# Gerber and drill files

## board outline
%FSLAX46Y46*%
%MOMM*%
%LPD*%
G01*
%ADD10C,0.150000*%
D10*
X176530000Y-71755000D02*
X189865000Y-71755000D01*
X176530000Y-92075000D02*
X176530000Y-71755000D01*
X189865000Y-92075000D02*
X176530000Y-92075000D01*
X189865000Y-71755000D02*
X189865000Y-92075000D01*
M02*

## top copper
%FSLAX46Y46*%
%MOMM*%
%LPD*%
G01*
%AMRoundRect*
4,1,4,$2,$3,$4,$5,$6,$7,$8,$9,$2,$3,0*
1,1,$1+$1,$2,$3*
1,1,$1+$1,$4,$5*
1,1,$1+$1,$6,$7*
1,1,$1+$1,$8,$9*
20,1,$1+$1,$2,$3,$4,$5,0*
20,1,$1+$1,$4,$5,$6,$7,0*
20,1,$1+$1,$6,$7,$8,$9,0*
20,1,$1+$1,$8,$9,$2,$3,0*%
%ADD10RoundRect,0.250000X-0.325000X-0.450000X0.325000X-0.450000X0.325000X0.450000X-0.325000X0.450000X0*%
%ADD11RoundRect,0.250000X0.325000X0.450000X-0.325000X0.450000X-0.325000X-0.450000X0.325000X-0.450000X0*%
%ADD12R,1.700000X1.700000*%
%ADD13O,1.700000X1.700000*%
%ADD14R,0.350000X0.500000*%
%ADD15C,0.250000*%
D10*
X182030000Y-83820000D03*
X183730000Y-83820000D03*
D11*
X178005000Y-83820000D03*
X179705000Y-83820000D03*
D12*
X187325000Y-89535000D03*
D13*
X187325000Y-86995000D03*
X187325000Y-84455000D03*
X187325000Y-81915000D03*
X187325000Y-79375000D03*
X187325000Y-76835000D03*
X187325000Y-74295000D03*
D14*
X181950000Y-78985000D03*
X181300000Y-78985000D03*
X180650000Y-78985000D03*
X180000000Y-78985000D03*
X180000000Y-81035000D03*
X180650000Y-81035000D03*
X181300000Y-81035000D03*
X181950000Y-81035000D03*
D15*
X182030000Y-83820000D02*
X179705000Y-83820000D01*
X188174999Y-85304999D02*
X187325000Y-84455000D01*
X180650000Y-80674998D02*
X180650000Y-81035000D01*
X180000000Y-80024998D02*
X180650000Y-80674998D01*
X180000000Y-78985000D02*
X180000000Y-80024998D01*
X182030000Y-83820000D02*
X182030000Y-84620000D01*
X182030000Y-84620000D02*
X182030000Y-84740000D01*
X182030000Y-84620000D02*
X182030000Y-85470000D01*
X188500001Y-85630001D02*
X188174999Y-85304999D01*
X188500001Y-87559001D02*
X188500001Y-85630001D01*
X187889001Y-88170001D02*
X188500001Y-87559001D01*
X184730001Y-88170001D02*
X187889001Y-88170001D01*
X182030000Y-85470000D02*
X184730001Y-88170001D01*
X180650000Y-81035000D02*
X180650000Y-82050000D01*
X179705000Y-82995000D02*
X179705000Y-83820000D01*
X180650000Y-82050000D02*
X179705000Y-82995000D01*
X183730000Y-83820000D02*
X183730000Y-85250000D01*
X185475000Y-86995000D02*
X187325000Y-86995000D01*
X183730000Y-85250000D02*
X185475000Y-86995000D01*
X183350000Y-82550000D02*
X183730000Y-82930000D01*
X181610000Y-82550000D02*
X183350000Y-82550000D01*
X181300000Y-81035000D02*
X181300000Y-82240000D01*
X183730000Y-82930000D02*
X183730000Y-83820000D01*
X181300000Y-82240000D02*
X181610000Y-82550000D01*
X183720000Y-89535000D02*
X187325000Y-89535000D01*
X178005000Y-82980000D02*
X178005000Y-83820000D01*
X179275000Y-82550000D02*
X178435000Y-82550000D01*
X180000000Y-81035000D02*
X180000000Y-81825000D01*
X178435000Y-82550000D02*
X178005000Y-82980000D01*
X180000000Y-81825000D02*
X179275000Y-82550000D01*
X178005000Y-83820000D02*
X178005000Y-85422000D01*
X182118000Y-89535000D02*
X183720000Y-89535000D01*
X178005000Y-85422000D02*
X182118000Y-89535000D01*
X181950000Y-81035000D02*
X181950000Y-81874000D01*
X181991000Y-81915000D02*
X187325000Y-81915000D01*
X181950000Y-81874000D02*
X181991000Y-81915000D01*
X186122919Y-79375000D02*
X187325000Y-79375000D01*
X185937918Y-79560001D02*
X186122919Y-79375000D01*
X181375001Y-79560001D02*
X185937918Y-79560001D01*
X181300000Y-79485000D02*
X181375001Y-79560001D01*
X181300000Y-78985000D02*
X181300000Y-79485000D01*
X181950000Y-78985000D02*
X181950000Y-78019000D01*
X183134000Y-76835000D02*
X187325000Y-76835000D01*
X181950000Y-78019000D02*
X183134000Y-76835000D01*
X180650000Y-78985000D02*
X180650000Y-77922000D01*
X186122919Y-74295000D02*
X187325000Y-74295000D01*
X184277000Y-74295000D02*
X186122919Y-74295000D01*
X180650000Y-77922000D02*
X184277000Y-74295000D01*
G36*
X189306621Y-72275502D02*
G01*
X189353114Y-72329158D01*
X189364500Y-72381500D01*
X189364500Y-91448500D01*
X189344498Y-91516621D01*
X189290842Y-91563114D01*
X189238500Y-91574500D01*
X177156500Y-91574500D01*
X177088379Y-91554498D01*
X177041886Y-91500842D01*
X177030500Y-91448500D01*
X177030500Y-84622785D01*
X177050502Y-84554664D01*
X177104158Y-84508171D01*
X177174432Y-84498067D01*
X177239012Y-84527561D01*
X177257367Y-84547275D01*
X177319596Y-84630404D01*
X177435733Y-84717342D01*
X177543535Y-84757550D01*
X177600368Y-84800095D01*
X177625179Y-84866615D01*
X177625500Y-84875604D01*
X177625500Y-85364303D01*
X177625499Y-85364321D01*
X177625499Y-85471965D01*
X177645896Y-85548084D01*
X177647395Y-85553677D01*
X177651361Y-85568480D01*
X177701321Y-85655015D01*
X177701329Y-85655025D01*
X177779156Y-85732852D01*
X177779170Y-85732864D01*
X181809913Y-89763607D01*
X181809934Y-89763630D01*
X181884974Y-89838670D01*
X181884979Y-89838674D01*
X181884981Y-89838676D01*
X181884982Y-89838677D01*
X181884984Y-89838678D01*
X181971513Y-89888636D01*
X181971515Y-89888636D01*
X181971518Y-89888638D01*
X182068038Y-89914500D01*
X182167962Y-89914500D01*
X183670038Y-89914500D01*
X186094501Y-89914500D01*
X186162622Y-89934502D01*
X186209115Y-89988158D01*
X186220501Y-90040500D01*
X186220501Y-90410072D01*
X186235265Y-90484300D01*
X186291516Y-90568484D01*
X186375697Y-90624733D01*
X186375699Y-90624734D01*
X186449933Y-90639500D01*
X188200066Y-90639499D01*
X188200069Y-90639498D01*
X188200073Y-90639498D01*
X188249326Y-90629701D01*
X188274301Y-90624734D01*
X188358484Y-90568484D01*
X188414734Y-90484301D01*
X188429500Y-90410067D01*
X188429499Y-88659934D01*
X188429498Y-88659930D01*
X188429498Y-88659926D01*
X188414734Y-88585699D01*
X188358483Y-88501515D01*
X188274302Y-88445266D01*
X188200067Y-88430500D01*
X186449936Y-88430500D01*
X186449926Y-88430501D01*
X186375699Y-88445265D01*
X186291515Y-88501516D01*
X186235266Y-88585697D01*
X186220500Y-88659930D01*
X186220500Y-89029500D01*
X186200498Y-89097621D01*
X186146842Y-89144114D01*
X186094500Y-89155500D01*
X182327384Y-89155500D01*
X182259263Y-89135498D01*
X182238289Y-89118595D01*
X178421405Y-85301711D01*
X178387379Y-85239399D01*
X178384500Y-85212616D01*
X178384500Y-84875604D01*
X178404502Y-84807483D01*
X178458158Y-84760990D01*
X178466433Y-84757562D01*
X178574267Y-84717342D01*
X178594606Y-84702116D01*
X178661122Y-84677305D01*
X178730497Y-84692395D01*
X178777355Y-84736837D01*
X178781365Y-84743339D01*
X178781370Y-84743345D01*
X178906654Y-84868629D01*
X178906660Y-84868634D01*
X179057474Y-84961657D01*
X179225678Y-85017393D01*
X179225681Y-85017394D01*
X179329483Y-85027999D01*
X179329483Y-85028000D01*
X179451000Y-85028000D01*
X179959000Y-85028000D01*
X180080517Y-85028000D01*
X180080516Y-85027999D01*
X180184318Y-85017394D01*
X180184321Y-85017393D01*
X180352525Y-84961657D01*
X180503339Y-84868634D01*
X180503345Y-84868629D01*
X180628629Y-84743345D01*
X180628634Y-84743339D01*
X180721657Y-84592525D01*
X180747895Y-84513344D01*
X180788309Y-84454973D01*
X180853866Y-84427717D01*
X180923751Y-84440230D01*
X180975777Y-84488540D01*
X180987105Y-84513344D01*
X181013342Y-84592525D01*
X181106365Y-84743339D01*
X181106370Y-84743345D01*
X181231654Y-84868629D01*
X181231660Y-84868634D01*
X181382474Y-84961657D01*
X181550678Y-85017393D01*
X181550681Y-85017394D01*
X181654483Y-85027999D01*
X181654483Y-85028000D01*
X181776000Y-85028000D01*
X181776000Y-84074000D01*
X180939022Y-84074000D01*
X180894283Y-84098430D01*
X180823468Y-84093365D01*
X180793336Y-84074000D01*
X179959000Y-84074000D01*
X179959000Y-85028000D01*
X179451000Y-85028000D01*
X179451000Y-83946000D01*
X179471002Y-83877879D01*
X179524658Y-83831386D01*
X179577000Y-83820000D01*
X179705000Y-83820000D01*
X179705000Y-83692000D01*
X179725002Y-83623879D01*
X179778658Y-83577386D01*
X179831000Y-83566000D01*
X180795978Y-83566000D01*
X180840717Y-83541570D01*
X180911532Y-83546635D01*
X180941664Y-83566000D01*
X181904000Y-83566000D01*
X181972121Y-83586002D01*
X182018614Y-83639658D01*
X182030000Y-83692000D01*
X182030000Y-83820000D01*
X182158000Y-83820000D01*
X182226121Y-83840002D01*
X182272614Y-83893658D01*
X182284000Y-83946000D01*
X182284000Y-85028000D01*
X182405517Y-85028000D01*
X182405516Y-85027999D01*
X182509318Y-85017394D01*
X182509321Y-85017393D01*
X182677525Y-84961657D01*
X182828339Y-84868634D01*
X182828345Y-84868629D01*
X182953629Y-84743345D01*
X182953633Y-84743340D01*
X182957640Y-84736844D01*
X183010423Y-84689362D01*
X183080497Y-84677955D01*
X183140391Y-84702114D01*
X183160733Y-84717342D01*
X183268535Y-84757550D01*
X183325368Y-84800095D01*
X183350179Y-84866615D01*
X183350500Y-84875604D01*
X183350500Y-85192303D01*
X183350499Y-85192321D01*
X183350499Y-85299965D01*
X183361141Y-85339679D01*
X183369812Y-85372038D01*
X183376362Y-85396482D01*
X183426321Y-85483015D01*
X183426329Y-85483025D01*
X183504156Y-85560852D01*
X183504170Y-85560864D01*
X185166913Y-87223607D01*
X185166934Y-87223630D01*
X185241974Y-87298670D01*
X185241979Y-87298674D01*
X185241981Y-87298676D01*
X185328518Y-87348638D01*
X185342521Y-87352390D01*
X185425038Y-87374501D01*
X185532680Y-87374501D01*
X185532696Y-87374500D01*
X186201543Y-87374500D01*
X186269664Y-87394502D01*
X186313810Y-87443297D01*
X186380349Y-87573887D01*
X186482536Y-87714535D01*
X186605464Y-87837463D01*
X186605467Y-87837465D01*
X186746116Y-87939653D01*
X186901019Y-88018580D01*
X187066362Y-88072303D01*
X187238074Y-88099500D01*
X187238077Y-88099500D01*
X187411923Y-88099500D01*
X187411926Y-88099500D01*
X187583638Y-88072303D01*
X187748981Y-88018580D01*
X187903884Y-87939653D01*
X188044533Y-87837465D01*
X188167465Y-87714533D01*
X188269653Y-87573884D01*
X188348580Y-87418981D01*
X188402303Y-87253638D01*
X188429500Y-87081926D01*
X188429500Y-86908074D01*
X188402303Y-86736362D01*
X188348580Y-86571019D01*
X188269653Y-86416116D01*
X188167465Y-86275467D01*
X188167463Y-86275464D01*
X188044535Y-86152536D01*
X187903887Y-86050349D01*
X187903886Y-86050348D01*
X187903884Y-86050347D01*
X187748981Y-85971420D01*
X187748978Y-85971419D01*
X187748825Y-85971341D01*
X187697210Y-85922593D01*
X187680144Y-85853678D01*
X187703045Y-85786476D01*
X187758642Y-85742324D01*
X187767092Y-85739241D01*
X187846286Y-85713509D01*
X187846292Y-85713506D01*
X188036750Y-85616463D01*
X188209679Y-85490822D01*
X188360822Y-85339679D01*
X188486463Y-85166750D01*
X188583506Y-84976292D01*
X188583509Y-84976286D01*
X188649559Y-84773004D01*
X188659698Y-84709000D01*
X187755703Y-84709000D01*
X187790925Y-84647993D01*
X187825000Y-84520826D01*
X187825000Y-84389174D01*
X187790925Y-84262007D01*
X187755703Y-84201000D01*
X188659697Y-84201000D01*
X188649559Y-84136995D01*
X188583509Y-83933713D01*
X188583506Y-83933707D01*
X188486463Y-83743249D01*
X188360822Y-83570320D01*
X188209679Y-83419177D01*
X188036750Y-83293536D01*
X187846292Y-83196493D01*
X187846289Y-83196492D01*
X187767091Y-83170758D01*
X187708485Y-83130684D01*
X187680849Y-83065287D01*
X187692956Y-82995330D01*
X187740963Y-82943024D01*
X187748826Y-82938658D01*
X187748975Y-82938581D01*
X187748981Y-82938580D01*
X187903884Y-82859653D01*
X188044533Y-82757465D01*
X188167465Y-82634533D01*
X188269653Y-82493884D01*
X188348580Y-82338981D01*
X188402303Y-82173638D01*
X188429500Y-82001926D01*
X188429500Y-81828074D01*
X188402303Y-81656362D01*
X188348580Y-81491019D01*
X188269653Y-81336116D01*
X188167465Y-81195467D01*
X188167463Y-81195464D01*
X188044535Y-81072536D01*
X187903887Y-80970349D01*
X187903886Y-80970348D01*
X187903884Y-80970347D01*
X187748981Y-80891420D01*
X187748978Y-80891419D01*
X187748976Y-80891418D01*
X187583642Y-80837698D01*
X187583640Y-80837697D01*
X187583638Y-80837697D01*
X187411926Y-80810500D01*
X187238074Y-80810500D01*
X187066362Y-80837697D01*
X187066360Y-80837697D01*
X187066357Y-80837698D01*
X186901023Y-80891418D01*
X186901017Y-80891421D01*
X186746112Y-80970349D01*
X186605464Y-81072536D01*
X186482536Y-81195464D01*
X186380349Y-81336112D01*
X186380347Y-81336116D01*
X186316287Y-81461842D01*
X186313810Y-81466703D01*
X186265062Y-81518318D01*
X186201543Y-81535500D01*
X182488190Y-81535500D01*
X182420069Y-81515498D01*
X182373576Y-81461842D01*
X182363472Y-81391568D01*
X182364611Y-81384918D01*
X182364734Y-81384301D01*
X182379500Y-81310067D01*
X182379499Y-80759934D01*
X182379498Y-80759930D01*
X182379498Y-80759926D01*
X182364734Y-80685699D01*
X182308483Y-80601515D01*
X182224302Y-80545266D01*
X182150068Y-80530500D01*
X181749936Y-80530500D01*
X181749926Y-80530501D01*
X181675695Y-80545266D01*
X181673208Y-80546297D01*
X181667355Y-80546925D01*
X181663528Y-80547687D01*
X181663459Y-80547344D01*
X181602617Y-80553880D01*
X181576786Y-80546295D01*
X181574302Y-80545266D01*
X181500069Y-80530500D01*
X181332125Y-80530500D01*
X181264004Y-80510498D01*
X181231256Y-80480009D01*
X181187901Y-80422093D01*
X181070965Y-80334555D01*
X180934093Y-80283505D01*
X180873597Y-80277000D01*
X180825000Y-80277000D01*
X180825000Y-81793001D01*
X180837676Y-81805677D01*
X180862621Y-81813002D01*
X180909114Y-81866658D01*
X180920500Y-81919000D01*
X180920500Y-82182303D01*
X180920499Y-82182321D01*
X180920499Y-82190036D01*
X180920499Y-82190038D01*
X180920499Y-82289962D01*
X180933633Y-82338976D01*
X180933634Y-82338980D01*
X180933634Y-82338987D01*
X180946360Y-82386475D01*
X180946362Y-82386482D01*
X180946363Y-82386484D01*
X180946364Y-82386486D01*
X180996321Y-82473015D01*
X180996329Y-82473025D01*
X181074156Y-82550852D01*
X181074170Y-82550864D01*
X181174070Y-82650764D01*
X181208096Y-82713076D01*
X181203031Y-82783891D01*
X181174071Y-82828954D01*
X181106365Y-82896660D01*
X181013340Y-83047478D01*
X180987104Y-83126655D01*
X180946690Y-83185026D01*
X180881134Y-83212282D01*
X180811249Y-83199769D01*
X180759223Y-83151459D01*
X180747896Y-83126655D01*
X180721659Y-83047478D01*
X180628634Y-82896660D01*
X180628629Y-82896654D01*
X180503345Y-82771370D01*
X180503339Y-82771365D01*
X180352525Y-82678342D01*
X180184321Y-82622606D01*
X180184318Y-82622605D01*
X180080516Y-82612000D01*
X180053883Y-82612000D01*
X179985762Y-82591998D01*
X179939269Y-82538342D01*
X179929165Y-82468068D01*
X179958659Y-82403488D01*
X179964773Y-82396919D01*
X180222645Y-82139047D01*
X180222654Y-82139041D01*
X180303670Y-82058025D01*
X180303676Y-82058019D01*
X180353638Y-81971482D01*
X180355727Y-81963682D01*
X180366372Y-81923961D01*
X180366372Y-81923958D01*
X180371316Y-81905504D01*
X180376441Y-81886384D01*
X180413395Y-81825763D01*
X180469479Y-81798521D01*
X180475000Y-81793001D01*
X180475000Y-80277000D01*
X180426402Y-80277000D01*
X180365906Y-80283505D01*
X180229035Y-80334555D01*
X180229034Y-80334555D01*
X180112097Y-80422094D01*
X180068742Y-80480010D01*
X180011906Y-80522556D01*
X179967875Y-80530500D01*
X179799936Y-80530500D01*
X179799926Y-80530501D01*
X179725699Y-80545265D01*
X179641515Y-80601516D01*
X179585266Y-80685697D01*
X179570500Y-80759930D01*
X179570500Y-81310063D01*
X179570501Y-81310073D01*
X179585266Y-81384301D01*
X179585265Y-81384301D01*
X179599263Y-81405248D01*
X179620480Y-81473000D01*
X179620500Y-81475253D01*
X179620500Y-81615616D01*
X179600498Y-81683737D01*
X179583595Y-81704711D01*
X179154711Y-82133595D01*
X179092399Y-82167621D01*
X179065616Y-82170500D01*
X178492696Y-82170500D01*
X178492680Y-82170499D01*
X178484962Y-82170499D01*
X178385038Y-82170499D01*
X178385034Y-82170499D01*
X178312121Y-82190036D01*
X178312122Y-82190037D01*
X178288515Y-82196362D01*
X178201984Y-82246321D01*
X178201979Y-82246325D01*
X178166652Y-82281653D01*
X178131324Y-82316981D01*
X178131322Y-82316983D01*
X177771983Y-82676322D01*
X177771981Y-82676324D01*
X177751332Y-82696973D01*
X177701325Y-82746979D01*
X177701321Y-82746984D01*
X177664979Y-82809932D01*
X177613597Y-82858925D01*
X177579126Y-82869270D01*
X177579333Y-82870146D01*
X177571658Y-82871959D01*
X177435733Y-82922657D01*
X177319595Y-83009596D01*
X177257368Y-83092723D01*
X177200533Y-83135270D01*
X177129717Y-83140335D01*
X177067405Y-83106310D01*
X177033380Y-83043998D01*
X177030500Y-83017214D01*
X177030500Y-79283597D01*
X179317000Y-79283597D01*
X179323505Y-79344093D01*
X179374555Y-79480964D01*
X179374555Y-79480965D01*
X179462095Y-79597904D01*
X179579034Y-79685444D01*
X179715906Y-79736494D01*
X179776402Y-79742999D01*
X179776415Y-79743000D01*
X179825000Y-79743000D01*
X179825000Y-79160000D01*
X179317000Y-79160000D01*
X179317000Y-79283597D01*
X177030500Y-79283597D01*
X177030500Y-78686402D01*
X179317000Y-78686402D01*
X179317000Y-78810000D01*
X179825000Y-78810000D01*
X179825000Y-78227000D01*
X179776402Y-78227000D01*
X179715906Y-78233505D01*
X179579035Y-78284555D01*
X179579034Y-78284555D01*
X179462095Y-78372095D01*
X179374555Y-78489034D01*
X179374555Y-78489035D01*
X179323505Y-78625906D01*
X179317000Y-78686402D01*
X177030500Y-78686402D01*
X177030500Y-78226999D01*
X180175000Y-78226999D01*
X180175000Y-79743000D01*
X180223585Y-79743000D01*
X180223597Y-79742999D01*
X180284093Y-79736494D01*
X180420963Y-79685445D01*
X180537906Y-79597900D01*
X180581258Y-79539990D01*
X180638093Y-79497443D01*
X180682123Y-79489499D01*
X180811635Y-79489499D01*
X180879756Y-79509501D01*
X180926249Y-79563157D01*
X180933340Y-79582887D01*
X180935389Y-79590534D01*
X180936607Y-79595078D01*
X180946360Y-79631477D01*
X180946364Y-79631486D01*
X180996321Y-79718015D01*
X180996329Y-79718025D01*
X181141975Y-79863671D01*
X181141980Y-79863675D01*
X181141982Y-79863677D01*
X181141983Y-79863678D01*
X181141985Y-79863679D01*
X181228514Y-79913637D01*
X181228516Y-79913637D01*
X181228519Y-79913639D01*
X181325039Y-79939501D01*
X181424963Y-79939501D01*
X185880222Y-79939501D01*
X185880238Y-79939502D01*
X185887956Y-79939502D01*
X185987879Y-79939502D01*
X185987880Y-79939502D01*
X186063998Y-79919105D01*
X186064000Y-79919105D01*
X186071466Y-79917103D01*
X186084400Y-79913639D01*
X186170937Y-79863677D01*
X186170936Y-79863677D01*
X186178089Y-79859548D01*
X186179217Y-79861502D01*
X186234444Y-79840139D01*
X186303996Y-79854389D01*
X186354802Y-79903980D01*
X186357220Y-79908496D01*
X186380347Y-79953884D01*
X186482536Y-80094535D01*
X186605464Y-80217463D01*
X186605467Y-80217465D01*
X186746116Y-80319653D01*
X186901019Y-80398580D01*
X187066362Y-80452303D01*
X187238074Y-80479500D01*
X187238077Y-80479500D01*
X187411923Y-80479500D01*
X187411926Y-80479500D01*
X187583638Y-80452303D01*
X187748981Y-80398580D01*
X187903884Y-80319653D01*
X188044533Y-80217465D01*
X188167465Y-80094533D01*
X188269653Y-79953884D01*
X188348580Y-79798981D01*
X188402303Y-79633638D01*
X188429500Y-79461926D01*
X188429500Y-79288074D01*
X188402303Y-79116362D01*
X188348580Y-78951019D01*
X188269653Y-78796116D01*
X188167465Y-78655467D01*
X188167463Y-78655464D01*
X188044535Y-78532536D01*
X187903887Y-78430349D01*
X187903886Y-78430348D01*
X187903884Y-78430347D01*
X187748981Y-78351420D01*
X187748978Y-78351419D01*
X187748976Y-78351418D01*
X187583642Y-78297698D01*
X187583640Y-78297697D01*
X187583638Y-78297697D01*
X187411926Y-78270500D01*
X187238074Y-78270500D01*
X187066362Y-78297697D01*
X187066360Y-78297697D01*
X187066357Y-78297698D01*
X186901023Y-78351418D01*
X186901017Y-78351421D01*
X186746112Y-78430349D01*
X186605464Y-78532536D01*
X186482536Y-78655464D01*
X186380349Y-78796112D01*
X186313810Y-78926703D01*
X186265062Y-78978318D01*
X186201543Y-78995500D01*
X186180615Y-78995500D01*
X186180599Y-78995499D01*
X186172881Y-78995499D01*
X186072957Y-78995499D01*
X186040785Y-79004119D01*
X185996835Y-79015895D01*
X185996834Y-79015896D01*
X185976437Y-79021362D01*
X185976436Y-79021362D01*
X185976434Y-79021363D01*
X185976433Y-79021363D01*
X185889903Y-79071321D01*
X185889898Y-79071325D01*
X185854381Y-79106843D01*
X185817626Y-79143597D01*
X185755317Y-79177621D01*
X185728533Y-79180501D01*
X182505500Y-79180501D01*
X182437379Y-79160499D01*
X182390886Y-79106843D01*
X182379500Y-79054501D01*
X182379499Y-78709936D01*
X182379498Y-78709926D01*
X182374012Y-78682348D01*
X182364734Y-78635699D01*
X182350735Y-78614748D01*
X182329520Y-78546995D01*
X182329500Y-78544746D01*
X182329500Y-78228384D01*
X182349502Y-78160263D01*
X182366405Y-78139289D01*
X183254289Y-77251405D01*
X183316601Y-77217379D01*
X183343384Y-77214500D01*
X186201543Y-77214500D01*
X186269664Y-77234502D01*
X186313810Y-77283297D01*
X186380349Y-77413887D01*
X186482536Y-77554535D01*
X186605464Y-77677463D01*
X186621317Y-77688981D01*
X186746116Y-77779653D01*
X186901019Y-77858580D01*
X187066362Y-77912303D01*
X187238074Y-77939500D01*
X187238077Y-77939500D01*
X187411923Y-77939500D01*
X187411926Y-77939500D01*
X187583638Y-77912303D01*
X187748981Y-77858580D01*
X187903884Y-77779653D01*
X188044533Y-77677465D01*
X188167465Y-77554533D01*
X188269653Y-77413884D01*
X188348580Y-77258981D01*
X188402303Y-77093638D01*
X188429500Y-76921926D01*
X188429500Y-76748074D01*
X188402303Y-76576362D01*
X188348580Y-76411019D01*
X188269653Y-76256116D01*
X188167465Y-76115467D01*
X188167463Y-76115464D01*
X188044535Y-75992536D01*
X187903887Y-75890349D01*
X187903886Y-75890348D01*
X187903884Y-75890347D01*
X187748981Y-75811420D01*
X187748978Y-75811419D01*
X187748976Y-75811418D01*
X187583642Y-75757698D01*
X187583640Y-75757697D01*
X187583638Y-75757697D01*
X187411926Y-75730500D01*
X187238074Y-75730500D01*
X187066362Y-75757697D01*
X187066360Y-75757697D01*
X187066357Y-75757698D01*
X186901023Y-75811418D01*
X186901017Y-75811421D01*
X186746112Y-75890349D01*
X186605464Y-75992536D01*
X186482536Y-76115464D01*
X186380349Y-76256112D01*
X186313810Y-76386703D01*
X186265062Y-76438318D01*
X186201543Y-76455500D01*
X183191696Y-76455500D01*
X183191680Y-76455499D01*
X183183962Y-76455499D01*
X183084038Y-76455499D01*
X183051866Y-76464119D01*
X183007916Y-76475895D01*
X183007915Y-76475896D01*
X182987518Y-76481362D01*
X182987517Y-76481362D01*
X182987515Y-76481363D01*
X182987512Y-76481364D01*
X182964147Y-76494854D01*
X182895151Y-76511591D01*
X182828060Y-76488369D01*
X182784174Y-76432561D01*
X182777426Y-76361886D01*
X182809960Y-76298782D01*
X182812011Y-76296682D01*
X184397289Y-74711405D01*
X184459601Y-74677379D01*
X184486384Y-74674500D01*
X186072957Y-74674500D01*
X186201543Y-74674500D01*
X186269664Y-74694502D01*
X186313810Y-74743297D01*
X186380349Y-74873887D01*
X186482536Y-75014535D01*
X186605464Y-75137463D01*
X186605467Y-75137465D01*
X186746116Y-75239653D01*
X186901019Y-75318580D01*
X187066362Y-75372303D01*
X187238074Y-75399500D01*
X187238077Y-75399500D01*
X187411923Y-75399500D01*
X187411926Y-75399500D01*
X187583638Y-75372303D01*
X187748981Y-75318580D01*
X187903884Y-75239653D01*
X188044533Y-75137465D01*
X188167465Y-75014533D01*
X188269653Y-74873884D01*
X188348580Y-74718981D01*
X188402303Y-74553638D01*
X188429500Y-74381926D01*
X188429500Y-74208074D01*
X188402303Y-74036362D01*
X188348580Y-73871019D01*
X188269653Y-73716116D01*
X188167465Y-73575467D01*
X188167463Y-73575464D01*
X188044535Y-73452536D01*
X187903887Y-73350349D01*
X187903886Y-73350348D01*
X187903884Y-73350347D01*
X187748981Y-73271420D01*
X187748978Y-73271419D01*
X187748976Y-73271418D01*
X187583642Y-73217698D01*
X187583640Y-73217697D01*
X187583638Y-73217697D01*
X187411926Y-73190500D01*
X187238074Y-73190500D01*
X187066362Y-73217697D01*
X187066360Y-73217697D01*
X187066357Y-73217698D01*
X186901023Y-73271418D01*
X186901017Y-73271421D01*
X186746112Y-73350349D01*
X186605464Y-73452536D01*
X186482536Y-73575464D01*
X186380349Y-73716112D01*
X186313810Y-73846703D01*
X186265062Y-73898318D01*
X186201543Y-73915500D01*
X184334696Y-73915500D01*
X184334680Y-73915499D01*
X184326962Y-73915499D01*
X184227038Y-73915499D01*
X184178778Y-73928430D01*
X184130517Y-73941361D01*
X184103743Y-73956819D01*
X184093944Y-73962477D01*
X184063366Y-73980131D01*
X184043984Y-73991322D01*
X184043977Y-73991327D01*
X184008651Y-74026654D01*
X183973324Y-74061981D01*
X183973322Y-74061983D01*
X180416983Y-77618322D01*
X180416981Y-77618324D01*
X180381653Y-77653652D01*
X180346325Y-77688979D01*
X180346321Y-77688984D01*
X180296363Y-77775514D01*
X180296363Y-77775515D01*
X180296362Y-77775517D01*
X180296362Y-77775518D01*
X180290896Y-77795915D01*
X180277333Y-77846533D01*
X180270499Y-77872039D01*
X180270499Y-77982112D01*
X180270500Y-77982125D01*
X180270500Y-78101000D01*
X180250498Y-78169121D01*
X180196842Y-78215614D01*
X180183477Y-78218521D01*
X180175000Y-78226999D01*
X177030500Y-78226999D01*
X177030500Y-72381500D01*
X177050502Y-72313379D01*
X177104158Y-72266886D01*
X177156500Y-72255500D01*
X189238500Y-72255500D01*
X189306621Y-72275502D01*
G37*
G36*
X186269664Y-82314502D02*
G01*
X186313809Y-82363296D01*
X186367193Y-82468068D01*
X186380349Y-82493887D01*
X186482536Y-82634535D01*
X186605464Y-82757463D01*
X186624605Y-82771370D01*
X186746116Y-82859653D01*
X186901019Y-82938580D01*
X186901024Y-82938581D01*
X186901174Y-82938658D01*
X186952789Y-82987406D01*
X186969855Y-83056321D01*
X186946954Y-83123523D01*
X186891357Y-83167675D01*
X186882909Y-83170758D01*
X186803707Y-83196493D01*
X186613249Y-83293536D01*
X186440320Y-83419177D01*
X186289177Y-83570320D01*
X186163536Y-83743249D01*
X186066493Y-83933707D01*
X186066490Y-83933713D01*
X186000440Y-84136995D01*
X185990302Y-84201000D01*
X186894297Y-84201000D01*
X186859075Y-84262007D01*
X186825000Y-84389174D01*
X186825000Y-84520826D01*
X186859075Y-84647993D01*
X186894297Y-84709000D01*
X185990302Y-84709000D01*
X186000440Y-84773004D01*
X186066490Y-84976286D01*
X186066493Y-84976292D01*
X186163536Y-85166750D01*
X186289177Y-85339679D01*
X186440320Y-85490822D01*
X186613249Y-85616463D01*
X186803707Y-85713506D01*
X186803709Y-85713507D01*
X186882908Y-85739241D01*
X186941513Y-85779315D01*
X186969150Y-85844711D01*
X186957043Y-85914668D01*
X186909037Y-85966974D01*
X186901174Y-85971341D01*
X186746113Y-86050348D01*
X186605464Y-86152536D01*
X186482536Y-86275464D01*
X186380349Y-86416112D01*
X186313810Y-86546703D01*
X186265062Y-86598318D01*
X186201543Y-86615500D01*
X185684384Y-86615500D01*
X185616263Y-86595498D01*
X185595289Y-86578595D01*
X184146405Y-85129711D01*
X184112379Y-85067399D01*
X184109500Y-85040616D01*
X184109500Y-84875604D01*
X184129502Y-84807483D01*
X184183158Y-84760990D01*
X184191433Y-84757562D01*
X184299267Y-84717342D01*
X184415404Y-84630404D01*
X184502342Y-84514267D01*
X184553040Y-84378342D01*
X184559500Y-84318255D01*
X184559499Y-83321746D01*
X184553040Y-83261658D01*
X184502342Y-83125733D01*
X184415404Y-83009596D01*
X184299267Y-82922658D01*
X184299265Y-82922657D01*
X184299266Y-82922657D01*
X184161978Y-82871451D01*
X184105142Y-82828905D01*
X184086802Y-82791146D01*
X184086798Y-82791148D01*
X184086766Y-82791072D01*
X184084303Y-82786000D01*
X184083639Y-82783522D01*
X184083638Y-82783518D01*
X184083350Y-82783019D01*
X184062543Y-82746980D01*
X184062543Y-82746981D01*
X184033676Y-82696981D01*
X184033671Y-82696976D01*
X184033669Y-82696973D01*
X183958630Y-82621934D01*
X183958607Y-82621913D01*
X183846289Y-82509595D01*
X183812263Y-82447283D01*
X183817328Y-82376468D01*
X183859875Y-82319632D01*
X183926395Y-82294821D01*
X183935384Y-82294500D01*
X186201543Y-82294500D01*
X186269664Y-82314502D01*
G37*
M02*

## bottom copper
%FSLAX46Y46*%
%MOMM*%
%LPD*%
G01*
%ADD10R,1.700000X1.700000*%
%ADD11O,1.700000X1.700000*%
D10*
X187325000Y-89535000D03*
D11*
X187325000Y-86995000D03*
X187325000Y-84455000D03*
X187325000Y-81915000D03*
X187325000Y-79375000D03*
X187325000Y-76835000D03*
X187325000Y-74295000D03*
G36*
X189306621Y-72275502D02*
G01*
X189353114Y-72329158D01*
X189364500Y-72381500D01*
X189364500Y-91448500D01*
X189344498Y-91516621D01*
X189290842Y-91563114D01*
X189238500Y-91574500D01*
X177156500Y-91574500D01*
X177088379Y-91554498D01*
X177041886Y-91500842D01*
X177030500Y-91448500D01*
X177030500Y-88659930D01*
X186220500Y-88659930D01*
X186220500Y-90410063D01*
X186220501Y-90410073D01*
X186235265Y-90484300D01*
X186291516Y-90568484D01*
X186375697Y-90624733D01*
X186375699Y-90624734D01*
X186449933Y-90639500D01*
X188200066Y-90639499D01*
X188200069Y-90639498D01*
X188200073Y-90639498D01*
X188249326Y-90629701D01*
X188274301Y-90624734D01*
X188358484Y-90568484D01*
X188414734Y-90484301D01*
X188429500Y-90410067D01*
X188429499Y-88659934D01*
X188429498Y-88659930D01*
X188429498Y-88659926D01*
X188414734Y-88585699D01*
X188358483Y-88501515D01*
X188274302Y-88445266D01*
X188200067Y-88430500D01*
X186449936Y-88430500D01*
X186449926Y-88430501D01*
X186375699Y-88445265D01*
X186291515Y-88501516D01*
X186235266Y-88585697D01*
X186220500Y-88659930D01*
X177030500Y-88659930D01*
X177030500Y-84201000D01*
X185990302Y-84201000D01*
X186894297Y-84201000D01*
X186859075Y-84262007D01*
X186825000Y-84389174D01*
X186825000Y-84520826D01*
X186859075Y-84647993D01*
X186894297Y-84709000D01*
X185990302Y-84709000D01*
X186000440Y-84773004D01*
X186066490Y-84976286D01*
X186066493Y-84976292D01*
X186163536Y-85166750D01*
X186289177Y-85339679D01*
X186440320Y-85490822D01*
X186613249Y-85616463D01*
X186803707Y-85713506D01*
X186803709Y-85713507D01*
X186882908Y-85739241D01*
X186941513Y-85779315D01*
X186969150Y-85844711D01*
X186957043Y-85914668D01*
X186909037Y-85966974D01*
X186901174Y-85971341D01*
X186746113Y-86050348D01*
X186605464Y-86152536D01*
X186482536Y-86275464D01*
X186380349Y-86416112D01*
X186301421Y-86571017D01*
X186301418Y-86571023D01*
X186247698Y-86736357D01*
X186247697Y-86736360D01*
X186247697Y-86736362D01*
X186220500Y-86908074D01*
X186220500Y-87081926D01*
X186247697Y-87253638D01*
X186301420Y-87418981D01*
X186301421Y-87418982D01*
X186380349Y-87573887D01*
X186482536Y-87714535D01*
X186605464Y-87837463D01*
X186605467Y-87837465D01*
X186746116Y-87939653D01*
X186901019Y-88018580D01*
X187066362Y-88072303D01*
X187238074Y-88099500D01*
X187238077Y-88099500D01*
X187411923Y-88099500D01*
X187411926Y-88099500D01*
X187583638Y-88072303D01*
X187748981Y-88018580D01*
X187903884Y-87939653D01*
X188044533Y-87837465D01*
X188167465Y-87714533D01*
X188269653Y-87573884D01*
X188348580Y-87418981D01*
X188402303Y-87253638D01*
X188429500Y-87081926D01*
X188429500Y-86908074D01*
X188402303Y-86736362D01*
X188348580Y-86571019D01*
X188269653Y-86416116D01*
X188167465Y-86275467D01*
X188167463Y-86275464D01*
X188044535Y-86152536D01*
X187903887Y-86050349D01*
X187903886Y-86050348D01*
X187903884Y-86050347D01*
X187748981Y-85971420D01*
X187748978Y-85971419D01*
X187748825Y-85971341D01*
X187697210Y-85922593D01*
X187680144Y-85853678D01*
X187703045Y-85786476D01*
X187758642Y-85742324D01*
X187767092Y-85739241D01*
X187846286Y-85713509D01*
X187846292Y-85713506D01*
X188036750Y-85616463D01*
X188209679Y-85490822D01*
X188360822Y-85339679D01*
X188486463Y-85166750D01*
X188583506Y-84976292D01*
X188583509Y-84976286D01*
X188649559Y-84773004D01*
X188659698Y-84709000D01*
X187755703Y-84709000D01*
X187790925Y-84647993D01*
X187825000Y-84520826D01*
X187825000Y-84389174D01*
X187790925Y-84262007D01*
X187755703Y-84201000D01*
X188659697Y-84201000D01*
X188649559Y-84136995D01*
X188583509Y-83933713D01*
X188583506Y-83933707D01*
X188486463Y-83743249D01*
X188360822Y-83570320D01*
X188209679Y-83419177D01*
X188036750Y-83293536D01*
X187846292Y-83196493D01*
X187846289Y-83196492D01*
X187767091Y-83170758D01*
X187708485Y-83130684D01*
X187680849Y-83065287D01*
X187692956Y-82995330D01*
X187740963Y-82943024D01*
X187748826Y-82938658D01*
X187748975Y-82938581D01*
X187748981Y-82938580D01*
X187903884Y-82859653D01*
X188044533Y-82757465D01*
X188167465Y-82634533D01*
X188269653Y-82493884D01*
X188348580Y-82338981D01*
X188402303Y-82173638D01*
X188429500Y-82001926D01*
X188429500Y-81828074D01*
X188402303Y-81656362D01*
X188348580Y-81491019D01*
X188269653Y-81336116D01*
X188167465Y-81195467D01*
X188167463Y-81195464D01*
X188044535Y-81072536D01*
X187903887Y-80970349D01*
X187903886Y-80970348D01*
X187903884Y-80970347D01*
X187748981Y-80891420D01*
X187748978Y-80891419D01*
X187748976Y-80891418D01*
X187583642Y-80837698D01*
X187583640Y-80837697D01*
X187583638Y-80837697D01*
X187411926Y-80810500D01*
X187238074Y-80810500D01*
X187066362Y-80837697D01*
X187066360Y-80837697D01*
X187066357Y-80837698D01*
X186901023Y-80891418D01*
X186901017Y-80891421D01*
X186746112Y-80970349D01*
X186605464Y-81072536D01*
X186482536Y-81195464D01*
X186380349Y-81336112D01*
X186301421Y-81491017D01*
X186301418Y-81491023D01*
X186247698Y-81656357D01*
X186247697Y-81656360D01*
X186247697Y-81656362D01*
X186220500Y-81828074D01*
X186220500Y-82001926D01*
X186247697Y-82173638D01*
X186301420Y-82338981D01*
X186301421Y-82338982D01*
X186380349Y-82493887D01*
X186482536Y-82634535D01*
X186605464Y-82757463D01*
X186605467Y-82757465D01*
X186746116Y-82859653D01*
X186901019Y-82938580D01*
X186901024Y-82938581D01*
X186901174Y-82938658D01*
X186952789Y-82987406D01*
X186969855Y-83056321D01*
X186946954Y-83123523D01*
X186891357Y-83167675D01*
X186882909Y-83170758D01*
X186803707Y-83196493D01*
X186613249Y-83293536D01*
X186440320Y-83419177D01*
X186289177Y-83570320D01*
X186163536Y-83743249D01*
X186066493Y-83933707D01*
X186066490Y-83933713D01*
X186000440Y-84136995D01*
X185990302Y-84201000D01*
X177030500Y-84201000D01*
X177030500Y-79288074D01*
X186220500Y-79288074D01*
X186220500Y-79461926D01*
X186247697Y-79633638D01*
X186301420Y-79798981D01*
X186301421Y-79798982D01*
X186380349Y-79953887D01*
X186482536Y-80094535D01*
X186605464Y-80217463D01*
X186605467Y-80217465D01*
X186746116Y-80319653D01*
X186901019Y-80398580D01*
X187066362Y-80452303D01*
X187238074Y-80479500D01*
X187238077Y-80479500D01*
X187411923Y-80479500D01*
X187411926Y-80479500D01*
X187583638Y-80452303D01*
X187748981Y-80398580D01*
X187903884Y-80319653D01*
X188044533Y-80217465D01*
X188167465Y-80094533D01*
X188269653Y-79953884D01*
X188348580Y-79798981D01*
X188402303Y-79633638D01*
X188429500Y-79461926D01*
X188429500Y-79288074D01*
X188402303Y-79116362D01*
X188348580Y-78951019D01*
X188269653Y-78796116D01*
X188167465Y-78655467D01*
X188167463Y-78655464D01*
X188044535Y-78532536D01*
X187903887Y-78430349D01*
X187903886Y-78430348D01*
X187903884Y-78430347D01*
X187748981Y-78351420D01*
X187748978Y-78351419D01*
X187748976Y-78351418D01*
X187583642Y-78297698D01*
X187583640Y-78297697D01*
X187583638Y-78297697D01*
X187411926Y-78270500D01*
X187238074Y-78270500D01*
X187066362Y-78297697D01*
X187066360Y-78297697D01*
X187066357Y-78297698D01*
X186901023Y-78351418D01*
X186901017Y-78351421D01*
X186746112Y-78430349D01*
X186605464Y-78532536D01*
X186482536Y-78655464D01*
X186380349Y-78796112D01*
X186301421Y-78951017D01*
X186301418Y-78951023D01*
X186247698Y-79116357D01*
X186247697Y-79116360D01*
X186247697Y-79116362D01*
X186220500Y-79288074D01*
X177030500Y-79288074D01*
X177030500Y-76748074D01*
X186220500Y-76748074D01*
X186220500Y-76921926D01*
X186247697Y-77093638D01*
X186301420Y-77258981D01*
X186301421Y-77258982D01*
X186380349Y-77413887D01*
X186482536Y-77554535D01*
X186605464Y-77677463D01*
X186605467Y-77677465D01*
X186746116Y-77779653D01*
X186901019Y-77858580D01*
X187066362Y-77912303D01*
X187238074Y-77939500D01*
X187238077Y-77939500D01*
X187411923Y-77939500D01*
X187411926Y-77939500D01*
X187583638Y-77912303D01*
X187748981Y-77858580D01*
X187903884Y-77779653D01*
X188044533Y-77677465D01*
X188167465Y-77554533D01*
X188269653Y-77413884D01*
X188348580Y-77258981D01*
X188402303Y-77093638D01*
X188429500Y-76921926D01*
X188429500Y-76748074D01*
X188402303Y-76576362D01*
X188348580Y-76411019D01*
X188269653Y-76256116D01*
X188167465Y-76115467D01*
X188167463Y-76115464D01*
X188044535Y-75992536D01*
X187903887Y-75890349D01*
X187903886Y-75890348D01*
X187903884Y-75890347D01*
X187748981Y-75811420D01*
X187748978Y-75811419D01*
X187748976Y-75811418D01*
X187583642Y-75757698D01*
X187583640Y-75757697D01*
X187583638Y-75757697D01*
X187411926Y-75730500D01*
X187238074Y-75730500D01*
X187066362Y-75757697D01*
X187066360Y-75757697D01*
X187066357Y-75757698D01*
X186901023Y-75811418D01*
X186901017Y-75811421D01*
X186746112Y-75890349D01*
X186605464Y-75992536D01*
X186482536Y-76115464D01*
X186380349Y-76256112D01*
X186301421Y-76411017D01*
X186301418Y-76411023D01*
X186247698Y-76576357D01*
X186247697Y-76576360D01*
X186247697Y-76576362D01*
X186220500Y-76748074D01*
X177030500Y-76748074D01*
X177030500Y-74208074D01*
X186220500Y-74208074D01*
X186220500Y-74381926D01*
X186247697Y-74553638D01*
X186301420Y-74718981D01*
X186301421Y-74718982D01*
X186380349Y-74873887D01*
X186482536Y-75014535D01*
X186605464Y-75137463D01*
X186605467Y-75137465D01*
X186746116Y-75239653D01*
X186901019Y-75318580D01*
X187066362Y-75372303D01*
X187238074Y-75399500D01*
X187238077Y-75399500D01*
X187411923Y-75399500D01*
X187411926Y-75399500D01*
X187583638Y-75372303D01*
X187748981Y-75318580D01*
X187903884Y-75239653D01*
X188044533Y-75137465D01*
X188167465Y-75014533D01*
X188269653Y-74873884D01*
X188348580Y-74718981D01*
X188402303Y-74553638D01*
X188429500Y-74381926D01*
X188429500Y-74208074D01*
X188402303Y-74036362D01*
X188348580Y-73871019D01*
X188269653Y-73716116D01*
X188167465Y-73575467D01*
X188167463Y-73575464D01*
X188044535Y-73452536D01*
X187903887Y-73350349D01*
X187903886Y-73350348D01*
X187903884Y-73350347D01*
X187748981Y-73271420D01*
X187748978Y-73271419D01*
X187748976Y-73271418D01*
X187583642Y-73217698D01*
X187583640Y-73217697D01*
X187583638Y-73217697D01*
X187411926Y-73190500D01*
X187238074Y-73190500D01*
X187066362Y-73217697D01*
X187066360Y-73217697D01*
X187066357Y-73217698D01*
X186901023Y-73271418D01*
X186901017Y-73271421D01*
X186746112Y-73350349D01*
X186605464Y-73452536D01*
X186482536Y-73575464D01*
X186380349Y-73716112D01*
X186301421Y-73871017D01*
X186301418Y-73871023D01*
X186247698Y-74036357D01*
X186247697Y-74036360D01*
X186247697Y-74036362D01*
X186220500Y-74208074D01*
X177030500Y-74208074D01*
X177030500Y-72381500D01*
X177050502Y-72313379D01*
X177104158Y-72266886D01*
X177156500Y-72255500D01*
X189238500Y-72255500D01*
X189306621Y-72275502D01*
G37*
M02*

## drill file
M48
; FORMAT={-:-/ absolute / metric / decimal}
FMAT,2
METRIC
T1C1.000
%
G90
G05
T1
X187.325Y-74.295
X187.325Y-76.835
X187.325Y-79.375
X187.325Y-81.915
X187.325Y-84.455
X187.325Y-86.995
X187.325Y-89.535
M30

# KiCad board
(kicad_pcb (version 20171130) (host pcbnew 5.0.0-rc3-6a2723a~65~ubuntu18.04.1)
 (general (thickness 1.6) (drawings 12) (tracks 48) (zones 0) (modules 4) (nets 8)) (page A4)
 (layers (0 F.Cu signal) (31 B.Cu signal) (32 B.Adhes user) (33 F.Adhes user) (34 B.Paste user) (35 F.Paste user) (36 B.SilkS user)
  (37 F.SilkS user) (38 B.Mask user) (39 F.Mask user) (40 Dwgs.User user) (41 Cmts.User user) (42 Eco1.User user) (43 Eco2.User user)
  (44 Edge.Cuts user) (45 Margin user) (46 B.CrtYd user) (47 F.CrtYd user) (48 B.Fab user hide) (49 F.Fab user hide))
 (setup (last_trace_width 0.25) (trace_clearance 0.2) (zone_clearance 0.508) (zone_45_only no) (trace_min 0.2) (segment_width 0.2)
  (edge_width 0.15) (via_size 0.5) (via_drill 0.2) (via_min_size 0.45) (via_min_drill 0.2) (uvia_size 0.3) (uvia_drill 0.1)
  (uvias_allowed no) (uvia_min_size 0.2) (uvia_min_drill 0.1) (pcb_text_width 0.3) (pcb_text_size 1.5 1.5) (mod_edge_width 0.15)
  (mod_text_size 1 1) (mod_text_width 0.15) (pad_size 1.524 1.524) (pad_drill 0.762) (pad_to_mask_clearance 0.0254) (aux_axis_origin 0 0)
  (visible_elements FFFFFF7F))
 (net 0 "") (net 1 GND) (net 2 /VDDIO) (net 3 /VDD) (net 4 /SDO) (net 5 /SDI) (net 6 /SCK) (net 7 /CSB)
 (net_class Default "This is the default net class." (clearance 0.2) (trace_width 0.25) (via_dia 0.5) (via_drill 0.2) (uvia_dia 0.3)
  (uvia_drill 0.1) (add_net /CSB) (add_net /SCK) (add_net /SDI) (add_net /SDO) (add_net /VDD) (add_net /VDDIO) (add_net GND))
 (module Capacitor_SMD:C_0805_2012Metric (layer F.Cu) (at 182.88 83.82)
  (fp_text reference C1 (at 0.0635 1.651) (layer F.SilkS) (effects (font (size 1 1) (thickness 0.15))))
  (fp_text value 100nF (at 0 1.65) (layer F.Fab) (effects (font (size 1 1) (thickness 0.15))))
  (pad 1 smd roundrect (at -0.85 0) (size 1.15 1.4) (layers F.Cu F.Paste F.Mask) (roundrect_rratio 0.217391) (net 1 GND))
  (pad 2 smd roundrect (at 0.85 0) (size 1.15 1.4) (layers F.Cu F.Paste F.Mask) (roundrect_rratio 0.217391) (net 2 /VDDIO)))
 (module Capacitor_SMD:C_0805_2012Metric (layer F.Cu) (at 178.855 83.82 180)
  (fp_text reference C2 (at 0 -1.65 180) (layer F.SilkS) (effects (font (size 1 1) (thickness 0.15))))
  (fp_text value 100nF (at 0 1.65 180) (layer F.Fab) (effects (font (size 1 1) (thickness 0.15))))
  (pad 2 smd roundrect (at 0.85 0 180) (size 1.15 1.4) (layers F.Cu F.Paste F.Mask) (roundrect_rratio 0.217391) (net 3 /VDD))
  (pad 1 smd roundrect (at -0.85 0 180) (size 1.15 1.4) (layers F.Cu F.Paste F.Mask) (roundrect_rratio 0.217391) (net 1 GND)))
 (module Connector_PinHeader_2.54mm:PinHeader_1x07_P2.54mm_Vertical (layer F.Cu) (at 187.325 89.535 180)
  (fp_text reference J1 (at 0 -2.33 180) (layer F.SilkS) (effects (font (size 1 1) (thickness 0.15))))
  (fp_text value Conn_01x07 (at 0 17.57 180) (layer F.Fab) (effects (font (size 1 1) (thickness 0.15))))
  (pad 1 thru_hole rect (at 0 0 180) (size 1.7 1.7) (drill 1) (layers *.Cu *.Mask) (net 3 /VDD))
  (pad 2 thru_hole oval (at 0 2.54 180) (size 1.7 1.7) (drill 1) (layers *.Cu *.Mask) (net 2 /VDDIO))
  (pad 3 thru_hole oval (at 0 5.08 180) (size 1.7 1.7) (drill 1) (layers *.Cu *.Mask) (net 1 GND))
  (pad 4 thru_hole oval (at 0 7.62 180) (size 1.7 1.7) (drill 1) (layers *.Cu *.Mask) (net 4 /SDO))
  (pad 5 thru_hole oval (at 0 10.16 180) (size 1.7 1.7) (drill 1) (layers *.Cu *.Mask) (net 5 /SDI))
  (pad 6 thru_hole oval (at 0 12.7 180) (size 1.7 1.7) (drill 1) (layers *.Cu *.Mask) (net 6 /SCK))
  (pad 7 thru_hole oval (at 0 15.24 180) (size 1.7 1.7) (drill 1) (layers *.Cu *.Mask) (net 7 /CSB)))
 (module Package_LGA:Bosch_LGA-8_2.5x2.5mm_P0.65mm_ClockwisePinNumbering (layer F.Cu) (at 180.975 80.01)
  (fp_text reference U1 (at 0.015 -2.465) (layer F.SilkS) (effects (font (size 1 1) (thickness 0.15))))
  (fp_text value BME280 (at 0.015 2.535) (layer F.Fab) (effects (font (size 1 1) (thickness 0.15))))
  (pad 4 smd rect (at 0.975 -1.025 90) (size 0.5 0.35) (layers F.Cu F.Paste F.Mask) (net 6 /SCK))
  (pad 3 smd rect (at 0.325 -1.025 90) (size 0.5 0.35) (layers F.Cu F.Paste F.Mask) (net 5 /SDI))
  (pad 2 smd rect (at -0.325 -1.025 90) (size 0.5 0.35) (layers F.Cu F.Paste F.Mask) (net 7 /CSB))
  (pad 1 smd rect (at -0.975 -1.025 90) (size 0.5 0.35) (layers F.Cu F.Paste F.Mask) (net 1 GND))
  (pad 8 smd rect (at -0.975 1.025 90) (size 0.5 0.35) (layers F.Cu F.Paste F.Mask) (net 3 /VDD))
  (pad 7 smd rect (at -0.325 1.025 90) (size 0.5 0.35) (layers F.Cu F.Paste F.Mask) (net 1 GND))
  (pad 6 smd rect (at 0.325 1.025 90) (size 0.5 0.35) (layers F.Cu F.Paste F.Mask) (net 2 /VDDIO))
  (pad 5 smd rect (at 0.975 1.025 90) (size 0.5 0.35) (layers F.Cu F.Paste F.Mask) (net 4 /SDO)))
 (gr_line (start 176.53 71.755) (end 189.865 71.755) (layer Edge.Cuts) (width 0.15))
 (gr_line (start 176.53 92.075) (end 176.53 71.755) (layer Edge.Cuts) (width 0.15))
 (gr_line (start 189.865 92.075) (end 176.53 92.075) (layer Edge.Cuts) (width 0.15))
 (gr_line (start 189.865 71.755) (end 189.865 92.075) (layer Edge.Cuts) (width 0.15))
 (segment (start 182.03 83.82) (end 179.705 83.82) (width 0.25) (layer F.Cu) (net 1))
 (segment (start 188.174999 85.304999) (end 187.325 84.455) (width 0.25) (layer F.Cu) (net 1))
 (segment (start 180.65 80.674998) (end 180.65 81.035) (width 0.25) (layer F.Cu) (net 1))
 (segment (start 180 80.024998) (end 180.65 80.674998) (width 0.25) (layer F.Cu) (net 1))
 (segment (start 180 78.985) (end 180 80.024998) (width 0.25) (layer F.Cu) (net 1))
 (segment (start 182.03 83.82) (end 182.03 84.62) (width 0.25) (layer F.Cu) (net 1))
 (segment (start 182.03 84.62) (end 182.03 84.74) (width 0.25) (layer F.Cu) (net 1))
 (segment (start 182.03 84.62) (end 182.03 85.47) (width 0.25) (layer F.Cu) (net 1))
 (segment (start 188.500001 85.630001) (end 188.174999 85.304999) (width 0.25) (layer F.Cu) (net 1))
 (segment (start 188.500001 87.559001) (end 188.500001 85.630001) (width 0.25) (layer F.Cu) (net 1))
 (segment (start 187.889001 88.170001) (end 188.500001 87.559001) (width 0.25) (layer F.Cu) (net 1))
 (segment (start 184.730001 88.170001) (end 187.889001 88.170001) (width 0.25) (layer F.Cu) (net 1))
 (segment (start 182.03 85.47) (end 184.730001 88.170001) (width 0.25) (layer F.Cu) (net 1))
 (segment (start 180.65 81.035) (end 180.65 82.05) (width 0.25) (layer F.Cu) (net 1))
 (segment (start 179.705 82.995) (end 179.705 83.82) (width 0.25) (layer F.Cu) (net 1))
 (segment (start 180.65 82.05) (end 179.705 82.995) (width 0.25) (layer F.Cu) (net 1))
 (segment (start 183.73 83.82) (end 183.73 85.25) (width 0.25) (layer F.Cu) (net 2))
 (segment (start 185.475 86.995) (end 187.325 86.995) (width 0.25) (layer F.Cu) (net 2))
 (segment (start 183.73 85.25) (end 185.475 86.995) (width 0.25) (layer F.Cu) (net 2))
 (segment (start 183.35 82.55) (end 183.73 82.93) (width 0.25) (layer F.Cu) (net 2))
 (segment (start 181.61 82.55) (end 183.35 82.55) (width 0.25) (layer F.Cu) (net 2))
 (segment (start 181.3 81.035) (end 181.3 82.24) (width 0.25) (layer F.Cu) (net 2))
 (segment (start 183.73 82.93) (end 183.73 83.82) (width 0.25) (layer F.Cu) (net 2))
 (segment (start 181.3 82.24) (end 181.61 82.55) (width 0.25) (layer F.Cu) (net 2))
 (segment (start 183.72 89.535) (end 187.325 89.535) (width 0.25) (layer F.Cu) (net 3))
 (segment (start 178.005 82.98) (end 178.005 83.82) (width 0.25) (layer F.Cu) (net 3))
 (segment (start 179.275 82.55) (end 178.435 82.55) (width 0.25) (layer F.Cu) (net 3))
 (segment (start 180 81.035) (end 180 81.825) (width 0.25) (layer F.Cu) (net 3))
 (segment (start 178.435 82.55) (end 178.005 82.98) (width 0.25) (layer F.Cu) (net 3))
 (segment (start 180 81.825) (end 179.275 82.55) (width 0.25) (layer F.Cu) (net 3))
 (segment (start 178.005 83.82) (end 178.005 85.422) (width 0.25) (layer F.Cu) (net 3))
 (segment (start 182.118 89.535) (end 183.72 89.535) (width 0.25) (layer F.Cu) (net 3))
 (segment (start 178.005 85.422) (end 182.118 89.535) (width 0.25) (layer F.Cu) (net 3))
 (segment (start 181.95 81.035) (end 181.95 81.874) (width 0.25) (layer F.Cu) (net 4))
 (segment (start 181.991 81.915) (end 187.325 81.915) (width 0.25) (layer F.Cu) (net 4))
 (segment (start 181.95 81.874) (end 181.991 81.915) (width 0.25) (layer F.Cu) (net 4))
 (segment (start 186.122919 79.375) (end 187.325 79.375) (width 0.25) (layer F.Cu) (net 5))
 (segment (start 185.937918 79.560001) (end 186.122919 79.375) (width 0.25) (layer F.Cu) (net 5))
 (segment (start 181.375001 79.560001) (end 185.937918 79.560001) (width 0.25) (layer F.Cu) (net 5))
 (segment (start 181.3 79.485) (end 181.375001 79.560001) (width 0.25) (layer F.Cu) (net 5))
 (segment (start 181.3 78.985) (end 181.3 79.485) (width 0.25) (layer F.Cu) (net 5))
 (segment (start 181.95 78.985) (end 181.95 78.019) (width 0.25) (layer F.Cu) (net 6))
 (segment (start 183.134 76.835) (end 187.325 76.835) (width 0.25) (layer F.Cu) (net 6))
 (segment (start 181.95 78.019) (end 183.134 76.835) (width 0.25) (layer F.Cu) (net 6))
 (segment (start 180.65 78.985) (end 180.65 77.922) (width 0.25) (layer F.Cu) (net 7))
 (segment (start 186.122919 74.295) (end 187.325 74.295) (width 0.25) (layer F.Cu) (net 7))
 (segment (start 184.277 74.295) (end 186.122919 74.295) (width 0.25) (layer F.Cu) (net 7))
 (segment (start 180.65 77.922) (end 184.277 74.295) (width 0.25) (layer F.Cu) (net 7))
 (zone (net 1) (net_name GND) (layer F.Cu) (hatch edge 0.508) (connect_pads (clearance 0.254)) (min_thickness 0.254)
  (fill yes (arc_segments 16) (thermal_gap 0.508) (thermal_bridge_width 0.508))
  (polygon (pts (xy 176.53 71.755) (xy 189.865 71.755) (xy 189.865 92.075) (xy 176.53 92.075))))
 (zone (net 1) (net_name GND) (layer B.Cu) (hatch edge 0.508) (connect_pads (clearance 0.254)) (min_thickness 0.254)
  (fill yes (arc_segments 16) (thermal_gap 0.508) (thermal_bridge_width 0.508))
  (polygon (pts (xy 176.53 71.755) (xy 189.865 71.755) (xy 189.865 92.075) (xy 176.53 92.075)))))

